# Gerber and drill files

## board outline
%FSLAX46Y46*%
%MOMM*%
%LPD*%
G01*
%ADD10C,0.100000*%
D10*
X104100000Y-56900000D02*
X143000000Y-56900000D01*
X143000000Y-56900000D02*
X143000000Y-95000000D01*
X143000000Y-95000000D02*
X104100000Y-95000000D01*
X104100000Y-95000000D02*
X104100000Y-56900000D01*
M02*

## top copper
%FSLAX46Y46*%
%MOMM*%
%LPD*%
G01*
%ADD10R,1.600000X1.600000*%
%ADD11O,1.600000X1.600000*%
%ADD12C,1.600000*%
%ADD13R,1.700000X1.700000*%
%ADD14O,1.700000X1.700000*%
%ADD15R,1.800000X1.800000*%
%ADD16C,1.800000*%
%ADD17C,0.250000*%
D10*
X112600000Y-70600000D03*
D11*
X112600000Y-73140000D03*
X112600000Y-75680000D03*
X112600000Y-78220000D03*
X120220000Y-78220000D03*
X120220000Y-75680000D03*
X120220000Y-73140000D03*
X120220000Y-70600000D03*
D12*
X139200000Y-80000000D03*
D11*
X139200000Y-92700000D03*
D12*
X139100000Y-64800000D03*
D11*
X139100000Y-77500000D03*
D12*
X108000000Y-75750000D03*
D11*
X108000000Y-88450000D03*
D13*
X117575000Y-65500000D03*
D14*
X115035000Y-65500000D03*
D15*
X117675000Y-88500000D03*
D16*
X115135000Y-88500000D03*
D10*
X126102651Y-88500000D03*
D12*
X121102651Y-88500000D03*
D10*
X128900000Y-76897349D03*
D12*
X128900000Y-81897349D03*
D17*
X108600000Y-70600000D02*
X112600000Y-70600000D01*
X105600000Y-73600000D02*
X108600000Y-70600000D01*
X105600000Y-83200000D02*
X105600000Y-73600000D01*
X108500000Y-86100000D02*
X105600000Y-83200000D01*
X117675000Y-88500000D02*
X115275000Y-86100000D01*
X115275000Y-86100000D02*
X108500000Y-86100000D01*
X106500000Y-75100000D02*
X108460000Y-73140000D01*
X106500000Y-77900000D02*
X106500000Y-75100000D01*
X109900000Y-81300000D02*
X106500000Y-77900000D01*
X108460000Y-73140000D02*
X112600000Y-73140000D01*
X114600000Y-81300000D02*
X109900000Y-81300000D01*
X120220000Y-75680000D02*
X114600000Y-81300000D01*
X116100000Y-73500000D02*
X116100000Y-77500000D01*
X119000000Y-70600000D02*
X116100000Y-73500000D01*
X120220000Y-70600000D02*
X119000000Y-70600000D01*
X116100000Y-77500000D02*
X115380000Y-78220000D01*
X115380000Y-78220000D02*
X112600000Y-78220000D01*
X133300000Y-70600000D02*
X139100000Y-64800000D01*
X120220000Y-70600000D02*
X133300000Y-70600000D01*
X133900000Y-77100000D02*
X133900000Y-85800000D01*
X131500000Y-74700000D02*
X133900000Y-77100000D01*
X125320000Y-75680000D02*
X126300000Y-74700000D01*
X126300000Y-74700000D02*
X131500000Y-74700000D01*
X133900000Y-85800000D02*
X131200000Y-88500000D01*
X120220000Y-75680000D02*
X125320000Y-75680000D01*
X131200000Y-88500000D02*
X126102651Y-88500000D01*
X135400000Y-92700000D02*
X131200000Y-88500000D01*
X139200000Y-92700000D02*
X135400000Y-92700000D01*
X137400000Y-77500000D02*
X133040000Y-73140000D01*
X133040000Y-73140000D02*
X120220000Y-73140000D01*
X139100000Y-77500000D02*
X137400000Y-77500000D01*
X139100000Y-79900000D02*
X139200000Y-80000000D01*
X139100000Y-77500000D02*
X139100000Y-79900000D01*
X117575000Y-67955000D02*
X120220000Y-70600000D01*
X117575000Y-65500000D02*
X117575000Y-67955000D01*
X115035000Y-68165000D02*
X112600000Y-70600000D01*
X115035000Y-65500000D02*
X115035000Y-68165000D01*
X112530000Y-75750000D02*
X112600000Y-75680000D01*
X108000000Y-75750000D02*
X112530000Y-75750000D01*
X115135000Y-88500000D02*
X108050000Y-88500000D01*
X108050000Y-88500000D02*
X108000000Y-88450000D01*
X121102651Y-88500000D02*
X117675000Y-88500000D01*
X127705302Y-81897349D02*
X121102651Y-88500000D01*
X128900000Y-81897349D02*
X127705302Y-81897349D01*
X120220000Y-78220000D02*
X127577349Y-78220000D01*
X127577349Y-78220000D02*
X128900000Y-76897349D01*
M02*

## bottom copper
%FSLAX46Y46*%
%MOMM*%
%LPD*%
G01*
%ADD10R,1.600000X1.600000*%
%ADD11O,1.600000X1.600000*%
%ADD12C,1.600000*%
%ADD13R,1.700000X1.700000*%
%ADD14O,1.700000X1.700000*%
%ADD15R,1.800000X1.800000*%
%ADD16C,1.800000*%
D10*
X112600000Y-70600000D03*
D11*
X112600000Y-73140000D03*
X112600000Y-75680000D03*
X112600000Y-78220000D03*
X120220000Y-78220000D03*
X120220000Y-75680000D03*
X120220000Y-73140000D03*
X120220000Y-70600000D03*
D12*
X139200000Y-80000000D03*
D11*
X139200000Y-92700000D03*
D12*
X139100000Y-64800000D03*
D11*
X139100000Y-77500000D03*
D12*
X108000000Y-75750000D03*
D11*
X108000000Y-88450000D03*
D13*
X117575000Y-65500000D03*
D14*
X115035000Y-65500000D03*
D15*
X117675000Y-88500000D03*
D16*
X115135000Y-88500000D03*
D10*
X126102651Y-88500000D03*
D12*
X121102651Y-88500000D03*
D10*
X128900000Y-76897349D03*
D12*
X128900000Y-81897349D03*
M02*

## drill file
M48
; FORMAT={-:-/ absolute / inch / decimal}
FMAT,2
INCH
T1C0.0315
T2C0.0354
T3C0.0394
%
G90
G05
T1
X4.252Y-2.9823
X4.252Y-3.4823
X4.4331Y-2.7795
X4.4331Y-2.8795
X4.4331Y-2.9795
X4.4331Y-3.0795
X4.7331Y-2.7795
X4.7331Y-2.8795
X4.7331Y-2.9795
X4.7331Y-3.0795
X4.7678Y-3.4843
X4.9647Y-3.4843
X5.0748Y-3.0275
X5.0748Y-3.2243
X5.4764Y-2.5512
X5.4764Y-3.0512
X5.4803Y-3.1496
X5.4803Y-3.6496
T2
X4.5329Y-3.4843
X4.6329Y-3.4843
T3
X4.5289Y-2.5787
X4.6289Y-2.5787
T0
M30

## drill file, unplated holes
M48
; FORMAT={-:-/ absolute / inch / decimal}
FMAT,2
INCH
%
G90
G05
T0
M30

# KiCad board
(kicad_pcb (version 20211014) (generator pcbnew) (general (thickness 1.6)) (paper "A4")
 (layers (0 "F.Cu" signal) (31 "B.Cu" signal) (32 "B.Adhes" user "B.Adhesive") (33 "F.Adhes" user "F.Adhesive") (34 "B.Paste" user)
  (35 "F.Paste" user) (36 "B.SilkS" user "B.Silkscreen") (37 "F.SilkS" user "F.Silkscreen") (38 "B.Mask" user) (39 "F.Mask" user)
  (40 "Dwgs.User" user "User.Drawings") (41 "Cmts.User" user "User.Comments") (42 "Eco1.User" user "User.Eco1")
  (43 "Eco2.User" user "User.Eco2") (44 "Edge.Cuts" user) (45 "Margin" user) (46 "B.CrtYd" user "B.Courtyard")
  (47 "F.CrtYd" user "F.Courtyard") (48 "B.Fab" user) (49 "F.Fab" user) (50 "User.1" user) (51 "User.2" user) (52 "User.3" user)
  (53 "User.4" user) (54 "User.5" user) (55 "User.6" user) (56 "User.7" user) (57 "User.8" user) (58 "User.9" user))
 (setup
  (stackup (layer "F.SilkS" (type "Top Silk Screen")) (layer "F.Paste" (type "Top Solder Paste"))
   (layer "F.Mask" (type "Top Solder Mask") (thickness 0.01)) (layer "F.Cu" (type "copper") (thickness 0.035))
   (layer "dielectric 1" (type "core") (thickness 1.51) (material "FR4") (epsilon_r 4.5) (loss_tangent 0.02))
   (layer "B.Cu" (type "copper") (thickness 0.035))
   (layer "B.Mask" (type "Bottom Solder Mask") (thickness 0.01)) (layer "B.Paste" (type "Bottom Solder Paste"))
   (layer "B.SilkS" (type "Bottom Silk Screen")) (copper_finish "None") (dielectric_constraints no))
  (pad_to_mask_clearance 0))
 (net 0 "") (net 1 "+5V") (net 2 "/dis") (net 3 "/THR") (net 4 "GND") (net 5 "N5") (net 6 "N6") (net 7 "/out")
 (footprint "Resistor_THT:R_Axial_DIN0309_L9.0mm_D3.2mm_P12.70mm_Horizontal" (layer "F.Cu") (at 139.1 64.8 -90)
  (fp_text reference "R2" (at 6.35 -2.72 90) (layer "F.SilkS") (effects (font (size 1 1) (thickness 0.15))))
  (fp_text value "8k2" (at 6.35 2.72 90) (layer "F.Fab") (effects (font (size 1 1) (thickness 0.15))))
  (pad "1" thru_hole circle (at 0 0 270) (size 1.6 1.6) (drill 0.8) (layers *.Cu *.Mask) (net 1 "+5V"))
  (pad "2" thru_hole oval (at 12.7 0 270) (size 1.6 1.6) (drill 0.8) (layers *.Cu *.Mask) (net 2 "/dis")))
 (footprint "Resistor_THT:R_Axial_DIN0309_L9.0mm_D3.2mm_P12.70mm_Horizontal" (layer "F.Cu") (at 139.2 80 -90)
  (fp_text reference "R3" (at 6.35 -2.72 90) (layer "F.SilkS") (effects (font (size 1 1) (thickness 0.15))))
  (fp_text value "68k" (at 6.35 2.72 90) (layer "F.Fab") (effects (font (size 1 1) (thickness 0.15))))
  (pad "1" thru_hole circle (at 0 0 270) (size 1.6 1.6) (drill 0.8) (layers *.Cu *.Mask) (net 2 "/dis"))
  (pad "2" thru_hole oval (at 12.7 0 270) (size 1.6 1.6) (drill 0.8) (layers *.Cu *.Mask) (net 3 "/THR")))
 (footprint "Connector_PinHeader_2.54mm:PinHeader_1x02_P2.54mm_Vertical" (layer "F.Cu") (at 117.575 65.5 -90)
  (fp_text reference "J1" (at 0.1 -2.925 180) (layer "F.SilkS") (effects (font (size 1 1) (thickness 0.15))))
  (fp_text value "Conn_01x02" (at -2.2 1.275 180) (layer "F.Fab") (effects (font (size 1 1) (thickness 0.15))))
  (pad "1" thru_hole rect (at 0 0 270) (size 1.7 1.7) (drill 1) (layers *.Cu *.Mask) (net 1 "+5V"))
  (pad "2" thru_hole oval (at 0 2.54 270) (size 1.7 1.7) (drill 1) (layers *.Cu *.Mask) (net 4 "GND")))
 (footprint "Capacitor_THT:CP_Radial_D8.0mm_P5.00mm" (layer "F.Cu") (at 126.102651 88.5 180)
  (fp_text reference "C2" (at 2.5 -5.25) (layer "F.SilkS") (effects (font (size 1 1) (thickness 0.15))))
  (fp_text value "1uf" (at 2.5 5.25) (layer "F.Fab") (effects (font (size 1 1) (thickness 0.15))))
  (pad "1" thru_hole rect (at 0 0 180) (size 1.6 1.6) (drill 0.8) (layers *.Cu *.Mask) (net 3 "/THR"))
  (pad "2" thru_hole circle (at 5 0 180) (size 1.6 1.6) (drill 0.8) (layers *.Cu *.Mask) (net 4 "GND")))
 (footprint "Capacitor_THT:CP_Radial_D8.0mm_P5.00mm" (layer "F.Cu") (at 128.9 76.897349 -90)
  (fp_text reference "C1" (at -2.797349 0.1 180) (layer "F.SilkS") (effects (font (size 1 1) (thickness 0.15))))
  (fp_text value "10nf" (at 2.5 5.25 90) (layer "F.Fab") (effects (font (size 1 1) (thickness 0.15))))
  (pad "1" thru_hole rect (at 0 0 270) (size 1.6 1.6) (drill 0.8) (layers *.Cu *.Mask) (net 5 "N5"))
  (pad "2" thru_hole circle (at 5 0 270) (size 1.6 1.6) (drill 0.8) (layers *.Cu *.Mask) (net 4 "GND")))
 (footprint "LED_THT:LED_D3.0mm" (layer "F.Cu") (at 117.675 88.5 180)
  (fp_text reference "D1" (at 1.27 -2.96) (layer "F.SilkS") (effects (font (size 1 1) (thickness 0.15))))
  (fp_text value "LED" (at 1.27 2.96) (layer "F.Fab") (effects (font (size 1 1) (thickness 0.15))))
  (pad "1" thru_hole rect (at 0 0 180) (size 1.8 1.8) (drill 0.9) (layers *.Cu *.Mask) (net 4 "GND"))
  (pad "2" thru_hole circle (at 2.54 0 180) (size 1.8 1.8) (drill 0.9) (layers *.Cu *.Mask) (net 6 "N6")))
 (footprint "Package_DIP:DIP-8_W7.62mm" (layer "F.Cu") (at 112.6 70.6)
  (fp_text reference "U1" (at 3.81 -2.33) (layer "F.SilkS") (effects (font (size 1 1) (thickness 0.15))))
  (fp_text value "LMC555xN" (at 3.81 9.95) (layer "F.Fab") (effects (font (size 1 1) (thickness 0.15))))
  (pad "1" thru_hole rect (at 0 0) (size 1.6 1.6) (drill 0.8) (layers *.Cu *.Mask) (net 4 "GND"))
  (pad "2" thru_hole oval (at 0 2.54) (size 1.6 1.6) (drill 0.8) (layers *.Cu *.Mask) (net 3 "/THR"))
  (pad "3" thru_hole oval (at 0 5.08) (size 1.6 1.6) (drill 0.8) (layers *.Cu *.Mask) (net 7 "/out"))
  (pad "4" thru_hole oval (at 0 7.62) (size 1.6 1.6) (drill 0.8) (layers *.Cu *.Mask) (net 1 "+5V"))
  (pad "5" thru_hole oval (at 7.62 7.62) (size 1.6 1.6) (drill 0.8) (layers *.Cu *.Mask) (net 5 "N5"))
  (pad "6" thru_hole oval (at 7.62 5.08) (size 1.6 1.6) (drill 0.8) (layers *.Cu *.Mask) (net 3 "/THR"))
  (pad "7" thru_hole oval (at 7.62 2.54) (size 1.6 1.6) (drill 0.8) (layers *.Cu *.Mask) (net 2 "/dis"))
  (pad "8" thru_hole oval (at 7.62 0) (size 1.6 1.6) (drill 0.8) (layers *.Cu *.Mask) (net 1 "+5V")))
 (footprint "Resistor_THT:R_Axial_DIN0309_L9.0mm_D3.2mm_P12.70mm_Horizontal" (layer "F.Cu") (at 108 75.75 -90)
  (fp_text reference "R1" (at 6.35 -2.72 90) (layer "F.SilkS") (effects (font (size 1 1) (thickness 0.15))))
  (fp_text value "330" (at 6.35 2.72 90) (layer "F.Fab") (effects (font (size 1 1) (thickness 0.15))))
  (pad "1" thru_hole circle (at 0 0 270) (size 1.6 1.6) (drill 0.8) (layers *.Cu *.Mask) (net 7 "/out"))
  (pad "2" thru_hole oval (at 12.7 0 270) (size 1.6 1.6) (drill 0.8) (layers *.Cu *.Mask) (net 6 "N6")))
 (gr_rect (start 104.1 56.9) (end 143 95) (layer "Edge.Cuts") (width 0.1) (fill none))
 (segment (start 127.577349 78.22) (end 128.9 76.897349) (width 0.25) (layer "F.Cu") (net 5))
 (segment (start 120.22 78.22) (end 127.577349 78.22) (width 0.25) (layer "F.Cu") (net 5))
 (segment (start 115.035 65.5) (end 115.035 68.165) (width 0.25) (layer "F.Cu") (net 4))
 (segment (start 128.9 81.897349) (end 127.705302 81.897349) (width 0.25) (layer "F.Cu") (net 4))
 (segment (start 105.6 83.2) (end 105.6 73.6) (width 0.25) (layer "F.Cu") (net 4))
 (segment (start 127.705302 81.897349) (end 121.102651 88.5) (width 0.25) (layer "F.Cu") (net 4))
 (segment (start 105.6 73.6) (end 108.6 70.6) (width 0.25) (layer "F.Cu") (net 4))
 (segment (start 115.275 86.1) (end 108.5 86.1) (width 0.25) (layer "F.Cu") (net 4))
 (segment (start 117.675 88.5) (end 115.275 86.1) (width 0.25) (layer "F.Cu") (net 4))
 (segment (start 115.035 68.165) (end 112.6 70.6) (width 0.25) (layer "F.Cu") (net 4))
 (segment (start 108.5 86.1) (end 105.6 83.2) (width 0.25) (layer "F.Cu") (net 4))
 (segment (start 121.102651 88.5) (end 117.675 88.5) (width 0.25) (layer "F.Cu") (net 4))
 (segment (start 108.6 70.6) (end 112.6 70.6) (width 0.25) (layer "F.Cu") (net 4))
 (segment (start 133.9 85.8) (end 131.2 88.5) (width 0.25) (layer "F.Cu") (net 3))
 (segment (start 131.5 74.7) (end 133.9 77.1) (width 0.25) (layer "F.Cu") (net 3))
 (segment (start 120.22 75.68) (end 125.32 75.68) (width 0.25) (layer "F.Cu") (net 3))
 (segment (start 108.46 73.14) (end 112.6 73.14) (width 0.25) (layer "F.Cu") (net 3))
 (segment (start 133.9 77.1) (end 133.9 85.8) (width 0.25) (layer "F.Cu") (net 3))
 (segment (start 114.6 81.3) (end 109.9 81.3) (width 0.25) (layer "F.Cu") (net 3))
 (segment (start 139.2 92.7) (end 135.4 92.7) (width 0.25) (layer "F.Cu") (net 3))
 (segment (start 125.32 75.68) (end 126.3 74.7) (width 0.25) (layer "F.Cu") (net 3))
 (segment (start 120.22 75.68) (end 114.6 81.3) (width 0.25) (layer "F.Cu") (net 3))
 (segment (start 131.2 88.5) (end 126.102651 88.5) (width 0.25) (layer "F.Cu") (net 3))
 (segment (start 135.4 92.7) (end 131.2 88.5) (width 0.25) (layer "F.Cu") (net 3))
 (segment (start 106.5 75.1) (end 108.46 73.14) (width 0.25) (layer "F.Cu") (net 3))
 (segment (start 126.3 74.7) (end 131.5 74.7) (width 0.25) (layer "F.Cu") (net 3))
 (segment (start 109.9 81.3) (end 106.5 77.9) (width 0.25) (layer "F.Cu") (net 3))
 (segment (start 106.5 77.9) (end 106.5 75.1) (width 0.25) (layer "F.Cu") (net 3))
 (segment (start 108.05 88.5) (end 108 88.45) (width 0.25) (layer "F.Cu") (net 6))
 (segment (start 115.135 88.5) (end 108.05 88.5) (width 0.25) (layer "F.Cu") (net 6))
 (segment (start 119 70.6) (end 116.1 73.5) (width 0.25) (layer "F.Cu") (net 1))
 (segment (start 120.22 70.6) (end 119 70.6) (width 0.25) (layer "F.Cu") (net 1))
 (segment (start 115.38 78.22) (end 112.6 78.22) (width 0.25) (layer "F.Cu") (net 1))
 (segment (start 116.1 73.5) (end 116.1 77.5) (width 0.25) (layer "F.Cu") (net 1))
 (segment (start 117.575 65.5) (end 117.575 67.955) (width 0.25) (layer "F.Cu") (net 1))
 (segment (start 133.3 70.6) (end 139.1 64.8) (width 0.25) (layer "F.Cu") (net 1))
 (segment (start 116.1 77.5) (end 115.38 78.22) (width 0.25) (layer "F.Cu") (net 1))
 (segment (start 120.22 70.6) (end 133.3 70.6) (width 0.25) (layer "F.Cu") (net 1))
 (segment (start 117.575 67.955) (end 120.22 70.6) (width 0.25) (layer "F.Cu") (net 1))
 (segment (start 108 75.75) (end 112.53 75.75) (width 0.25) (layer "F.Cu") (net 7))
 (segment (start 112.53 75.75) (end 112.6 75.68) (width 0.25) (layer "F.Cu") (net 7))
 (segment (start 137.4 77.5) (end 133.04 73.14) (width 0.25) (layer "F.Cu") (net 2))
 (segment (start 133.04 73.14) (end 120.22 73.14) (width 0.25) (layer "F.Cu") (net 2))
 (segment (start 139.1 77.5) (end 139.1 79.9) (width 0.25) (layer "F.Cu") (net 2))
 (segment (start 139.1 79.9) (end 139.2 80) (width 0.25) (layer "F.Cu") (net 2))
 (segment (start 139.1 77.5) (end 137.4 77.5) (width 0.25) (layer "F.Cu") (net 2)))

